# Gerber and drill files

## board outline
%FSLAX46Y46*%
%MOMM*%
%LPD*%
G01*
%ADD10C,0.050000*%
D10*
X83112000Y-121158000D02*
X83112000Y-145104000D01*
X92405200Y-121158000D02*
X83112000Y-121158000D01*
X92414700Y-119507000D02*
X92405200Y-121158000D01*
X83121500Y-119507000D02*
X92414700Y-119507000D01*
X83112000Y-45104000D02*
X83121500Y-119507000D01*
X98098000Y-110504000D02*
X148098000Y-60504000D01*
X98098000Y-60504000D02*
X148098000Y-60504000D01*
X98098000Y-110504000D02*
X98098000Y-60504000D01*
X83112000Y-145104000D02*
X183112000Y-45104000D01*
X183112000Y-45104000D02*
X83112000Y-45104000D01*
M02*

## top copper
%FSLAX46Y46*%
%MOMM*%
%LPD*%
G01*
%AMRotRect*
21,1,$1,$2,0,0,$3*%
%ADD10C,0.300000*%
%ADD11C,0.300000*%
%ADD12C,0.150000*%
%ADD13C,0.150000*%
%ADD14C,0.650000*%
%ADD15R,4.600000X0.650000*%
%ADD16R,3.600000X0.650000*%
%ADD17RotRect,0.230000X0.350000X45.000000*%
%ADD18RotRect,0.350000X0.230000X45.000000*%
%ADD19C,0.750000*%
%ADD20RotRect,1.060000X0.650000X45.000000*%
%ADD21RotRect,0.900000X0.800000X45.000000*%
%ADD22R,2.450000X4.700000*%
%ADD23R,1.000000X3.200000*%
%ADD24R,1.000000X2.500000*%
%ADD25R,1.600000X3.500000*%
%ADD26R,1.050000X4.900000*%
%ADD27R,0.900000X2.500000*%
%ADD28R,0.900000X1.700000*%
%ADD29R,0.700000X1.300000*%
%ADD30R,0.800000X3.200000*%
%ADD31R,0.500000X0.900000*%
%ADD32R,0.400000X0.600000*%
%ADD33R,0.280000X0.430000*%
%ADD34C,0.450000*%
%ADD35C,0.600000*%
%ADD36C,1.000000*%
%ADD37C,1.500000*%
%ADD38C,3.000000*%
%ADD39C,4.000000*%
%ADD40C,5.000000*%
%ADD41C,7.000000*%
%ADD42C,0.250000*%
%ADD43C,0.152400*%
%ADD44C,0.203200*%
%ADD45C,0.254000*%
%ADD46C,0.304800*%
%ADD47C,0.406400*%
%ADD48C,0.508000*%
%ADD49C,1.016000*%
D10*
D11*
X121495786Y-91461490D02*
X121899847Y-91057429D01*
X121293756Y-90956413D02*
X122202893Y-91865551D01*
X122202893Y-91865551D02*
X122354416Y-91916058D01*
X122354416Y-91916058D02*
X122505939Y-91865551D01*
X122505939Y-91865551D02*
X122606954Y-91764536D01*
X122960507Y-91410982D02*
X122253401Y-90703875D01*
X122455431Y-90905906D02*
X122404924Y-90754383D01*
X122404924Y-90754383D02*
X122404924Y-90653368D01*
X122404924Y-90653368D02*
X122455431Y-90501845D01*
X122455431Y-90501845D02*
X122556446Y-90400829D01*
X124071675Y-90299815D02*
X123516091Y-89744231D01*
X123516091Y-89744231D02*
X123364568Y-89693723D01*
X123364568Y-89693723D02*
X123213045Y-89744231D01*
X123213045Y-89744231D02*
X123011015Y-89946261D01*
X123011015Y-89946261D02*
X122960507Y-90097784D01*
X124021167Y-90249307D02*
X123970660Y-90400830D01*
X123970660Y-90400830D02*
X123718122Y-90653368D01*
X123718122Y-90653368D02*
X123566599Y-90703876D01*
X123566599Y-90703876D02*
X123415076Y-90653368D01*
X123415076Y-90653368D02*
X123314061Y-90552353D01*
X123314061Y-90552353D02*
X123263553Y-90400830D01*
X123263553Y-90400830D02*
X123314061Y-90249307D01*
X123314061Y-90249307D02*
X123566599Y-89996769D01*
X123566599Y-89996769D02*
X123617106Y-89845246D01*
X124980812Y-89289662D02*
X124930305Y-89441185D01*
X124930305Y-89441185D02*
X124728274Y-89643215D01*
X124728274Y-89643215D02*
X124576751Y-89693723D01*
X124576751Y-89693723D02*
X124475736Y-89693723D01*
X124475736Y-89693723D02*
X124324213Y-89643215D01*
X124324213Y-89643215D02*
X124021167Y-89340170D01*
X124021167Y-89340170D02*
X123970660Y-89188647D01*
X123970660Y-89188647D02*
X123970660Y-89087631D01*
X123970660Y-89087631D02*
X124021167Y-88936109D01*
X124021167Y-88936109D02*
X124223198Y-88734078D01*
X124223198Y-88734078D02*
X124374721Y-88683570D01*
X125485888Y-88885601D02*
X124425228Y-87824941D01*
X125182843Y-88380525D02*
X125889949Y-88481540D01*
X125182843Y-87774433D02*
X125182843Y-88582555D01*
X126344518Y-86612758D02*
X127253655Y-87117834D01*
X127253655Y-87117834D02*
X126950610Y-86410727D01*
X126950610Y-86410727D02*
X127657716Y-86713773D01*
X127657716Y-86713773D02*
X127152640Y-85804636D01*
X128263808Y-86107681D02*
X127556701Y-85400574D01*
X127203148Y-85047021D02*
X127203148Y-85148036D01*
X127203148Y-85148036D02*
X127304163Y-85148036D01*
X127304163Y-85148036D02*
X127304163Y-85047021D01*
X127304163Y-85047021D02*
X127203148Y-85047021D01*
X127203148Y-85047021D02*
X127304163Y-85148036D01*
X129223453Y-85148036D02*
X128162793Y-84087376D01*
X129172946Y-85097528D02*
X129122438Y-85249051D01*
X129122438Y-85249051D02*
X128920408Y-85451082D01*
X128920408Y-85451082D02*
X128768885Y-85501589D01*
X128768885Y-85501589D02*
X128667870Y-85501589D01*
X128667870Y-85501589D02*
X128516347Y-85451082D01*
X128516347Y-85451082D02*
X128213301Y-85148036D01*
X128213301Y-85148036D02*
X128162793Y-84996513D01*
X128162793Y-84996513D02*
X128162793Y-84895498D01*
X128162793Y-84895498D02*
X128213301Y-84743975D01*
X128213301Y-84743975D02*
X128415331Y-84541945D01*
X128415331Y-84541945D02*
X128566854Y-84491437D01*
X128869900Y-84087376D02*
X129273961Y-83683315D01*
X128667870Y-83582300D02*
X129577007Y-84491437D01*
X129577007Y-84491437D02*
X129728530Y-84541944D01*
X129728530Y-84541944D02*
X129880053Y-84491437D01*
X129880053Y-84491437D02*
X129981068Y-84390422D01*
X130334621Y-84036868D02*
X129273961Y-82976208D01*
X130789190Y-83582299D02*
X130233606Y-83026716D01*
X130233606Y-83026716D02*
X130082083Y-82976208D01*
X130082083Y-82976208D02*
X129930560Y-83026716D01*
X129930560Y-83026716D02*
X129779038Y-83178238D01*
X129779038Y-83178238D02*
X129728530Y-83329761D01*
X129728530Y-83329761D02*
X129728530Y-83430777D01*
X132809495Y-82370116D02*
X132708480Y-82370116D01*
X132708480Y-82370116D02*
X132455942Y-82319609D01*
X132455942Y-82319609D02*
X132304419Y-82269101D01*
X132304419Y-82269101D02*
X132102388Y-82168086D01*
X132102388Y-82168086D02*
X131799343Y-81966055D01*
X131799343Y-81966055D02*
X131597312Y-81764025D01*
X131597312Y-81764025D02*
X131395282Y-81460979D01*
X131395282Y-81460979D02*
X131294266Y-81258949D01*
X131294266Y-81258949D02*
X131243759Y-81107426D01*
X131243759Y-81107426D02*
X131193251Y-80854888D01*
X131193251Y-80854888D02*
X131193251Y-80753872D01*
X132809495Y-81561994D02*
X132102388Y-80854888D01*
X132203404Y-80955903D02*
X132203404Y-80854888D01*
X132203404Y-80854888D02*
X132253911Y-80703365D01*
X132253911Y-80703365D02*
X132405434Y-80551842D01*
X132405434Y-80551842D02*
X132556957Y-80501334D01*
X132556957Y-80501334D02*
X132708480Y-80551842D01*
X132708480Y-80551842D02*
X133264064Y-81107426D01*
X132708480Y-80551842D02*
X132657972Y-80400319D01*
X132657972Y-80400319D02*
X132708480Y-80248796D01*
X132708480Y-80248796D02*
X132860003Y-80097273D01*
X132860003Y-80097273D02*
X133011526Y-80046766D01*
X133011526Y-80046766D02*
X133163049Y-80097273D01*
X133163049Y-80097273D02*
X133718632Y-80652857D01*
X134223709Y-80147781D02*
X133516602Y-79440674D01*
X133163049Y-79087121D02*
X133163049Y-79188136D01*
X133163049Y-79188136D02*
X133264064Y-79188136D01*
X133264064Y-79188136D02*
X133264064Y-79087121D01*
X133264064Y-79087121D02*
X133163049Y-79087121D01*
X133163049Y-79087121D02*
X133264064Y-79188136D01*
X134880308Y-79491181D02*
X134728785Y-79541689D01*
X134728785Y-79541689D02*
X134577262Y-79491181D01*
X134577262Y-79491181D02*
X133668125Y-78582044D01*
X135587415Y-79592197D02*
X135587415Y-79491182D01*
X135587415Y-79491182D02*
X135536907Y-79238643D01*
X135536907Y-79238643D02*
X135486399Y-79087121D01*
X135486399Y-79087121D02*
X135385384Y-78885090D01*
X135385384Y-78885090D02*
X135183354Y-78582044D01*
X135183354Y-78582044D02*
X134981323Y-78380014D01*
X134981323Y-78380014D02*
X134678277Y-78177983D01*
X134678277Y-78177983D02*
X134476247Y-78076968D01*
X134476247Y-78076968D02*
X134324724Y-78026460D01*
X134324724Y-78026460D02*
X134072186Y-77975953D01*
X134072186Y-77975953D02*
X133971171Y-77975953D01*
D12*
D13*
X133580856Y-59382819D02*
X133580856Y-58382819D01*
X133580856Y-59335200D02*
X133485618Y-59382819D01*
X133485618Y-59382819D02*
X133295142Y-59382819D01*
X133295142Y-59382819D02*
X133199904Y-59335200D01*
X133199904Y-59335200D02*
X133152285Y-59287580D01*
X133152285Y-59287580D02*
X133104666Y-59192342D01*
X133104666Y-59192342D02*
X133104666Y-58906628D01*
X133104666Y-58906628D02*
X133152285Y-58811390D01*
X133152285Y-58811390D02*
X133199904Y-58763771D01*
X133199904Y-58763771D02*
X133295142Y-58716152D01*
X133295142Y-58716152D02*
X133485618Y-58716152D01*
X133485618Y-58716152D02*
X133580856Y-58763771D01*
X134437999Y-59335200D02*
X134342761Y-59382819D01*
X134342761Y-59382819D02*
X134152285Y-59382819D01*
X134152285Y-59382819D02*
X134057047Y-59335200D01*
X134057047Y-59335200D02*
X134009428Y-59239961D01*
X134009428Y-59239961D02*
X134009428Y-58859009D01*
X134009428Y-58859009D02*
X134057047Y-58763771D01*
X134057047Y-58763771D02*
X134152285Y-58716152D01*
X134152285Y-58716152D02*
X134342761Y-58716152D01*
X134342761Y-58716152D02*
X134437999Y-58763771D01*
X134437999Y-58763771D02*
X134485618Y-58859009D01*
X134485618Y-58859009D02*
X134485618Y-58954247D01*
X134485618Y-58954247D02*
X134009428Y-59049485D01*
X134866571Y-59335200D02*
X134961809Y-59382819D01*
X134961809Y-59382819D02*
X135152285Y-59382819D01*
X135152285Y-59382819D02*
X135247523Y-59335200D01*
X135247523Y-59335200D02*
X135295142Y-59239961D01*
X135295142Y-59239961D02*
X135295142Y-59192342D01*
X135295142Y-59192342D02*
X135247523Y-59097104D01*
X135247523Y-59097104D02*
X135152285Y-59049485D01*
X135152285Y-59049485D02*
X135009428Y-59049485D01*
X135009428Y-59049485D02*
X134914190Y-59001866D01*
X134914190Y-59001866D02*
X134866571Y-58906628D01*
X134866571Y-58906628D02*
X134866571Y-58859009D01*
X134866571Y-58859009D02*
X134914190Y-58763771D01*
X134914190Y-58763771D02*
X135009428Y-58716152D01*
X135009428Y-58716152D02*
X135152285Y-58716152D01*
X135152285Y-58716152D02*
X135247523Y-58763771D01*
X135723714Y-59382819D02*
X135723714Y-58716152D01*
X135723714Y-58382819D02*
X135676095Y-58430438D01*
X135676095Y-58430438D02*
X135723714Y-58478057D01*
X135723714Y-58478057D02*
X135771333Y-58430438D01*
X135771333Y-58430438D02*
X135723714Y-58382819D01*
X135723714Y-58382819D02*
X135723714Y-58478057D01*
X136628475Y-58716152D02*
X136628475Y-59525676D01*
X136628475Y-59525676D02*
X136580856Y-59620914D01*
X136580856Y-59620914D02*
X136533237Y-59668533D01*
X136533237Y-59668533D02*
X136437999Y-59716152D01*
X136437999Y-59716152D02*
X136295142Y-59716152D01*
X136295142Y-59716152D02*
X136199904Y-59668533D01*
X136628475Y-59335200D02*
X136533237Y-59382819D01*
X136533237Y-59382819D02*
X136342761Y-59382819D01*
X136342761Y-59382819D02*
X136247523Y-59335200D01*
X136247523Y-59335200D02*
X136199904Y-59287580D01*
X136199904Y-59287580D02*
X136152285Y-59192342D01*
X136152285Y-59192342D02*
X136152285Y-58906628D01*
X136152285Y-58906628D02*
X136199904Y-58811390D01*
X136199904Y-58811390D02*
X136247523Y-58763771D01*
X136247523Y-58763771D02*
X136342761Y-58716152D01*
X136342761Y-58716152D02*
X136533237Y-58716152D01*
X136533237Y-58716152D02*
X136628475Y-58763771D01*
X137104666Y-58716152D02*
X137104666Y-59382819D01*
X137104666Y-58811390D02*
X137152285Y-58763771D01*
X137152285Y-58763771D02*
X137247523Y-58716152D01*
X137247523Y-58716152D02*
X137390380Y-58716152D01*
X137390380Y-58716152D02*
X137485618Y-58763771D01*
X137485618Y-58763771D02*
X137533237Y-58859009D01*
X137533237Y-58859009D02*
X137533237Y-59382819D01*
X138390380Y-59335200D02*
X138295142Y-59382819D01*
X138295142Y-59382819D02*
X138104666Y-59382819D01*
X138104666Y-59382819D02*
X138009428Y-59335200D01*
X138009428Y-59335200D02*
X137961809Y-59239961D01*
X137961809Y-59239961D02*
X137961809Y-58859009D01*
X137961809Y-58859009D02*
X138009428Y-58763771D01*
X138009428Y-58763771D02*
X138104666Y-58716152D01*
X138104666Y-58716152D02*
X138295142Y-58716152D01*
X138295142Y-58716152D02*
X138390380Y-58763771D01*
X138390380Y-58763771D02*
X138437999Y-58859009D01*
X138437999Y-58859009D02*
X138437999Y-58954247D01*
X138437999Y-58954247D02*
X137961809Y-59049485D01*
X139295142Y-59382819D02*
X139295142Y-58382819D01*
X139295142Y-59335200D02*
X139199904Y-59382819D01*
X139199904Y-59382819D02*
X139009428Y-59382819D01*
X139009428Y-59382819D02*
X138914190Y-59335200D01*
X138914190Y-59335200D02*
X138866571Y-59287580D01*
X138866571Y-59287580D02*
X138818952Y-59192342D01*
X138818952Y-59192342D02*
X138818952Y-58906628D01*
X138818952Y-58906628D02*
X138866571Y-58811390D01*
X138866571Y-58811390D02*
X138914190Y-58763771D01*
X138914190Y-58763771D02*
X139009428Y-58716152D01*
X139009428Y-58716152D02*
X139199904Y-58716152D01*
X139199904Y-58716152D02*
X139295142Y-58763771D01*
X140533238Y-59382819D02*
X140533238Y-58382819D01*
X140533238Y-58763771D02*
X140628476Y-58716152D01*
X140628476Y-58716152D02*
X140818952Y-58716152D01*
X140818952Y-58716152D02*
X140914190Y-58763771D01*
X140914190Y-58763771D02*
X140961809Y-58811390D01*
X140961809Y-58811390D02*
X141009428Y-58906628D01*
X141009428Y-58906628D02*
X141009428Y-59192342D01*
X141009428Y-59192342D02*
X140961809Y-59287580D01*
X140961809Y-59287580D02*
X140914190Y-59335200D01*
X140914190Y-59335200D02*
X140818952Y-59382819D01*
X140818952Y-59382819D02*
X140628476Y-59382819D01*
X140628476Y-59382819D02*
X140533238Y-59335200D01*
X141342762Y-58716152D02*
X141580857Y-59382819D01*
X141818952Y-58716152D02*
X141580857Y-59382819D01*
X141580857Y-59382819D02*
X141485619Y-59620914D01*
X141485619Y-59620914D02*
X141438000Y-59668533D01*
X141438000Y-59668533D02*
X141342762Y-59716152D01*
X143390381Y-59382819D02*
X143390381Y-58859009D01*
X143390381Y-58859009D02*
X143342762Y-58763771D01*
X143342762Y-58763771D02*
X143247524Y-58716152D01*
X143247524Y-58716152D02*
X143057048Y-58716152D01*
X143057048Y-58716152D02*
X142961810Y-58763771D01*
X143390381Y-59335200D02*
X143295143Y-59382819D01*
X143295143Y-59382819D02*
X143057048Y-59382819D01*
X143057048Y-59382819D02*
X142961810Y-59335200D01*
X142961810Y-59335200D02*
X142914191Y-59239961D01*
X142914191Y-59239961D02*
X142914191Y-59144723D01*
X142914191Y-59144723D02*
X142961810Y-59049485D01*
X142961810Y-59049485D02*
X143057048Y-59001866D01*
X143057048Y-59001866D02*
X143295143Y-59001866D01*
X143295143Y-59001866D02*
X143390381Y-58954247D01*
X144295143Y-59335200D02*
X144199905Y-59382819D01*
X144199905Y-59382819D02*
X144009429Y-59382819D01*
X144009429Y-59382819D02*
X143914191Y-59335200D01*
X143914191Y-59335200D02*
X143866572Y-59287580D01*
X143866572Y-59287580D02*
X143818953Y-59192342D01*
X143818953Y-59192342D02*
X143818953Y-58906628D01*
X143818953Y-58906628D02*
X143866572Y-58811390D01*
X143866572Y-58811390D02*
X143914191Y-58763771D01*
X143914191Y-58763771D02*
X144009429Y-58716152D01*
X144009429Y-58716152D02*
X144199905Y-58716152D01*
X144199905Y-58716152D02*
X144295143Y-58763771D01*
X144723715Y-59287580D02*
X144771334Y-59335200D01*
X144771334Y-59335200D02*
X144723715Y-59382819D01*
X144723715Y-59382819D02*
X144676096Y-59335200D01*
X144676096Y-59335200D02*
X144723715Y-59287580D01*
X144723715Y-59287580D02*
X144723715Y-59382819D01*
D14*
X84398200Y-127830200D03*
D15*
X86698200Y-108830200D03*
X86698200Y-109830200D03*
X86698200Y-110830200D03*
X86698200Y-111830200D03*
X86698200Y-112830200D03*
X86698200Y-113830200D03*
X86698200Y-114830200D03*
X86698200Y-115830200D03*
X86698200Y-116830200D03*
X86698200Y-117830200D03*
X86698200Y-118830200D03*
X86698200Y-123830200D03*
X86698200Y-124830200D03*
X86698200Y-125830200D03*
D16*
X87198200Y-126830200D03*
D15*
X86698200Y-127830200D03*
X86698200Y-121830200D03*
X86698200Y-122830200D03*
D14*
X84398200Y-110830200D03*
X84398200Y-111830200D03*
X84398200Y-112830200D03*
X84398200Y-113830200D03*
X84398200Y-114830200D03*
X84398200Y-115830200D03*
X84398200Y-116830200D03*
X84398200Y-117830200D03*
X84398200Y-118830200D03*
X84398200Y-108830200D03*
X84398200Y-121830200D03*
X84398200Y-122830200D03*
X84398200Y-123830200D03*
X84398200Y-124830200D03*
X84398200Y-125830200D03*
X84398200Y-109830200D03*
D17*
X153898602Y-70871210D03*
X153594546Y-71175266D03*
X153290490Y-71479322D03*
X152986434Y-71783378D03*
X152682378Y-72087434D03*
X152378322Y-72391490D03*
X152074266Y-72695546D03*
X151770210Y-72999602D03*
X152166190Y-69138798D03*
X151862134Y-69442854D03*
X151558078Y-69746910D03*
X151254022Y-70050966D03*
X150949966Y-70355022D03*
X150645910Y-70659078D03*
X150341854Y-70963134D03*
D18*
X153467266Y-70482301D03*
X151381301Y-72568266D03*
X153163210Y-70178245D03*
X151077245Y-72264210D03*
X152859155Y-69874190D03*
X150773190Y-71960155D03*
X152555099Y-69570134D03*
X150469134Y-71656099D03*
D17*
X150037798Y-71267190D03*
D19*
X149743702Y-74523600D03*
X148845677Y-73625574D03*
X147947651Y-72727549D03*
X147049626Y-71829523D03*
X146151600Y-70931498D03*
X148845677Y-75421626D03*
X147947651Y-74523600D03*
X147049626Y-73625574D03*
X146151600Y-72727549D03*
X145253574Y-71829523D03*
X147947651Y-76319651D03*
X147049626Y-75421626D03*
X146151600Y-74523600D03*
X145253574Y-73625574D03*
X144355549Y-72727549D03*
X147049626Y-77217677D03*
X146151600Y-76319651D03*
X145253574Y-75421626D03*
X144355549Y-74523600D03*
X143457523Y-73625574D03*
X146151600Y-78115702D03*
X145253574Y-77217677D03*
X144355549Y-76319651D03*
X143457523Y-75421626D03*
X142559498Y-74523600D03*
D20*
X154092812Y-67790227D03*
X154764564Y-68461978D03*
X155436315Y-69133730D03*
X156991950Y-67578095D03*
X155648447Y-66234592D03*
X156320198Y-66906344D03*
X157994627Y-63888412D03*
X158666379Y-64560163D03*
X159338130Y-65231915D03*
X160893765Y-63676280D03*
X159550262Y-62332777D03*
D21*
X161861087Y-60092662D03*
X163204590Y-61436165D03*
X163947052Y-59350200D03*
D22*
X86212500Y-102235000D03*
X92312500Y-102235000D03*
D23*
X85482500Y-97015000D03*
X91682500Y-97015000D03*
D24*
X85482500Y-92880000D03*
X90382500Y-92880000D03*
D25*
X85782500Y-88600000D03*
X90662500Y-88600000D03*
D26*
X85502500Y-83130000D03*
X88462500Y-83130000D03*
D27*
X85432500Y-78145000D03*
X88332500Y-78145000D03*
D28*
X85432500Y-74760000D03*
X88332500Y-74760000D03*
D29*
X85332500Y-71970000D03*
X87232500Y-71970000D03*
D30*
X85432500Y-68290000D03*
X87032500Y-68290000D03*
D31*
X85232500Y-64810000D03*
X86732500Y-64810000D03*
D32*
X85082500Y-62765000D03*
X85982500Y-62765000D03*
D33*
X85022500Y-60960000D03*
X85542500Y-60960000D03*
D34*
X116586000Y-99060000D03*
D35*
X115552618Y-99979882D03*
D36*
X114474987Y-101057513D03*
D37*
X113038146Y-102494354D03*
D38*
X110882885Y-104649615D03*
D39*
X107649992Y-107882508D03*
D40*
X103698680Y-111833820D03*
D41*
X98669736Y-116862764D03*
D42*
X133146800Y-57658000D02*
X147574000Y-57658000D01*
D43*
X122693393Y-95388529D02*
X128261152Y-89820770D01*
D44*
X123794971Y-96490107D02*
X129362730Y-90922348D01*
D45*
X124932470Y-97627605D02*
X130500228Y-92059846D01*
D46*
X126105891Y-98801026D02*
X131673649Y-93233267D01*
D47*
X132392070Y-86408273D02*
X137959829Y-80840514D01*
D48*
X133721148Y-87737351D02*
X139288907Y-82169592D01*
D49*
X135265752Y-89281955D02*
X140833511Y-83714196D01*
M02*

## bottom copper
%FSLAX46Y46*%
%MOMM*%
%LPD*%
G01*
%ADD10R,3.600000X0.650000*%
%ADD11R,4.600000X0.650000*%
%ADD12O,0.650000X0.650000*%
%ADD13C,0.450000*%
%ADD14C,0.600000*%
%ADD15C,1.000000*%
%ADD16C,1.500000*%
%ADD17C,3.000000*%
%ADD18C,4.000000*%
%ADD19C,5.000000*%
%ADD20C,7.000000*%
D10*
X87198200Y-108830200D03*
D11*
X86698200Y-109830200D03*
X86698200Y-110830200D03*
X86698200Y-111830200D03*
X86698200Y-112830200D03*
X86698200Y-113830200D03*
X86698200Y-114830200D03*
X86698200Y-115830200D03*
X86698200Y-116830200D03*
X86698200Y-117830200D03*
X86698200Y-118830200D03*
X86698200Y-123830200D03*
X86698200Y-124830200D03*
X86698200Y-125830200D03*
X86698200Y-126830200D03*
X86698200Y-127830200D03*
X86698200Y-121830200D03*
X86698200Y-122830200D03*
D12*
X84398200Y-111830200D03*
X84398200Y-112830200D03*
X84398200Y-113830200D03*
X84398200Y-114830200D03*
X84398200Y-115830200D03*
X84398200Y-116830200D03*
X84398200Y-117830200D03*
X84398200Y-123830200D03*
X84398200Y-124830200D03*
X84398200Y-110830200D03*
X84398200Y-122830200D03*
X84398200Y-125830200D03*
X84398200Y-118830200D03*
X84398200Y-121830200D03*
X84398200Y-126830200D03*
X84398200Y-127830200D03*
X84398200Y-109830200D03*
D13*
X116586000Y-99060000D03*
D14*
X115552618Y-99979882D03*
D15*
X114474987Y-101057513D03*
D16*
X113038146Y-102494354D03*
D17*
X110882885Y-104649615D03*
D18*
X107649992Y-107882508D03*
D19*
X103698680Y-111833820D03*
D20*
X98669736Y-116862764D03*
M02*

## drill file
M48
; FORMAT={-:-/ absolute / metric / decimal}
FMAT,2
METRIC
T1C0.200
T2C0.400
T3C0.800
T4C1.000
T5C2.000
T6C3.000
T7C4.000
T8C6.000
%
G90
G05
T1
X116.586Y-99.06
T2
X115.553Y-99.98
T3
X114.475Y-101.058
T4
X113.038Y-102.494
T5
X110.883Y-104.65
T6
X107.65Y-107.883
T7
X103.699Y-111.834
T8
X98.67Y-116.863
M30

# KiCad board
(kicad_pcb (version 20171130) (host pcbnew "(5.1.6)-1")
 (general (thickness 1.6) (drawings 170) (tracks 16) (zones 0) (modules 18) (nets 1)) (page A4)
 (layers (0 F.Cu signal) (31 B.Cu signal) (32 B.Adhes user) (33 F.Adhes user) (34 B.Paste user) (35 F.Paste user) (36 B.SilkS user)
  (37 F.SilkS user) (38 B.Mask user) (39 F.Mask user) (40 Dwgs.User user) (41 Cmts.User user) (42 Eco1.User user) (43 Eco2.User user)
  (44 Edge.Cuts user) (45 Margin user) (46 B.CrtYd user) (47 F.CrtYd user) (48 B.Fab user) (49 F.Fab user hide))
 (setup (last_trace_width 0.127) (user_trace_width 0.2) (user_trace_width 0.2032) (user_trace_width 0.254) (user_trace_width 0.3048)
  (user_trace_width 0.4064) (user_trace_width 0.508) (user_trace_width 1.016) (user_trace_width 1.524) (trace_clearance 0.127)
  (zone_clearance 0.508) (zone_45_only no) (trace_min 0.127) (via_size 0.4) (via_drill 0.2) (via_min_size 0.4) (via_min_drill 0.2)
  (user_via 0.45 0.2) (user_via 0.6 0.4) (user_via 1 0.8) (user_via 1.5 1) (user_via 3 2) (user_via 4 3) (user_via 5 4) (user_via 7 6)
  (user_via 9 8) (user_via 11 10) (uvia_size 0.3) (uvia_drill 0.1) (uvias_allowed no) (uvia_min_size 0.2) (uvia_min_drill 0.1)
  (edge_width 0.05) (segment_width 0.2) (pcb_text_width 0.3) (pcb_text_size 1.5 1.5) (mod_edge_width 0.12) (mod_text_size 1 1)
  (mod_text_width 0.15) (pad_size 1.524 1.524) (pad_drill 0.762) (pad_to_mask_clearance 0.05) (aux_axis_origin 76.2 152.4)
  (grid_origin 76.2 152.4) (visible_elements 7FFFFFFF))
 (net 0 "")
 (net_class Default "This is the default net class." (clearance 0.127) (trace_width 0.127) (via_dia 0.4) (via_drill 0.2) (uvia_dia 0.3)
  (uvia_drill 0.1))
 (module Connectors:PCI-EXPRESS (layer F.Cu) (at 87.1982 108.8302 270)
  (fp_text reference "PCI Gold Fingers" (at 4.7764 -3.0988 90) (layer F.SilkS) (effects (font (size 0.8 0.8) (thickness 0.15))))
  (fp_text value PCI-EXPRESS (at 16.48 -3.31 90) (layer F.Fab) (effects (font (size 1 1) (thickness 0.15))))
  (pad "" connect circle (at 19 2.8 270) (size 0.65 0.65) (layers F.Cu F.Mask))
  (pad B1 connect rect (at 0 0.5 270) (size 0.65 4.6) (layers F.Cu F.Mask))
  (pad B2 connect rect (at 1 0.5 270) (size 0.65 4.6) (layers F.Cu F.Mask))
  (pad B3 connect rect (at 2 0.5 270) (size 0.65 4.6) (layers F.Cu F.Mask))
  (pad B4 connect rect (at 3 0.5 270) (size 0.65 4.6) (layers F.Cu F.Mask))
  (pad B5 connect rect (at 4 0.5 270) (size 0.65 4.6) (layers F.Cu F.Mask))
  (pad B6 connect rect (at 5 0.5 270) (size 0.65 4.6) (layers F.Cu F.Mask))
  (pad B7 connect rect (at 6 0.5 270) (size 0.65 4.6) (layers F.Cu F.Mask))
  (pad B8 connect rect (at 7 0.5 270) (size 0.65 4.6) (layers F.Cu F.Mask))
  (pad B9 connect rect (at 8 0.5 270) (size 0.65 4.6) (layers F.Cu F.Mask))
  (pad B10 connect rect (at 9 0.5 270) (size 0.65 4.6) (layers F.Cu F.Mask))
  (pad B11 connect rect (at 10 0.5 270) (size 0.65 4.6) (layers F.Cu F.Mask))
  (pad B14 connect rect (at 15 0.5 270) (size 0.65 4.6) (layers F.Cu F.Mask))
  (pad B15 connect rect (at 16 0.5 270) (size 0.65 4.6) (layers F.Cu F.Mask))
  (pad B16 connect rect (at 17 0.5 270) (size 0.65 4.6) (layers F.Cu F.Mask))
  (pad B17 connect rect (at 18 0 270) (size 0.65 3.6) (layers F.Cu F.Mask))
  (pad B18 connect rect (at 19 0.5 270) (size 0.65 4.6) (layers F.Cu F.Mask))
  (pad B12 connect rect (at 13 0.5 270) (size 0.65 4.6) (layers F.Cu F.Mask))
  (pad B13 connect rect (at 14 0.5 270) (size 0.65 4.6) (layers F.Cu F.Mask))
  (pad A1 connect rect (at 0 0 270) (size 0.65 3.6) (layers B.Cu B.Mask))
  (pad A2 connect rect (at 1 0.5 270) (size 0.65 4.6) (layers B.Cu B.Mask))
  (pad A3 connect rect (at 2 0.5 270) (size 0.65 4.6) (layers B.Cu B.Mask))
  (pad A4 connect rect (at 3 0.5 270) (size 0.65 4.6) (layers B.Cu B.Mask))
  (pad A5 connect rect (at 4 0.5 270) (size 0.65 4.6) (layers B.Cu B.Mask))
  (pad A6 connect rect (at 5 0.5 270) (size 0.65 4.6) (layers B.Cu B.Mask))
  (pad A7 connect rect (at 6 0.5 270) (size 0.65 4.6) (layers B.Cu B.Mask))
  (pad A8 connect rect (at 7 0.5 270) (size 0.65 4.6) (layers B.Cu B.Mask))
  (pad A9 connect rect (at 8 0.5 270) (size 0.65 4.6) (layers B.Cu B.Mask))
  (pad A10 connect rect (at 9 0.5 270) (size 0.65 4.6) (layers B.Cu B.Mask))
  (pad A11 connect rect (at 10 0.5 270) (size 0.65 4.6) (layers B.Cu B.Mask))
  (pad A14 connect rect (at 15 0.5 270) (size 0.65 4.6) (layers B.Cu B.Mask))
  (pad A15 connect rect (at 16 0.5 270) (size 0.65 4.6) (layers B.Cu B.Mask))
  (pad A16 connect rect (at 17 0.5 270) (size 0.65 4.6) (layers B.Cu B.Mask))
  (pad A17 connect rect (at 18 0.5 270) (size 0.65 4.6) (layers B.Cu B.Mask))
  (pad A18 connect rect (at 19 0.5 270) (size 0.65 4.6) (layers B.Cu B.Mask))
  (pad A12 connect rect (at 13 0.5 270) (size 0.65 4.6) (layers B.Cu B.Mask))
  (pad A13 connect rect (at 14 0.5 270) (size 0.65 4.6) (layers B.Cu B.Mask))
  (pad "" connect circle (at 2 2.8 270) (size 0.65 0.65) (layers F.Cu F.Mask))
  (pad "" connect circle (at 3 2.8 270) (size 0.65 0.65) (layers F.Cu F.Mask))
  (pad "" connect circle (at 4 2.8 270) (size 0.65 0.65) (layers F.Cu F.Mask))
  (pad "" connect circle (at 5 2.8 270) (size 0.65 0.65) (layers F.Cu F.Mask))
  (pad "" connect circle (at 6 2.8 270) (size 0.65 0.65) (layers F.Cu F.Mask))
  (pad "" connect circle (at 7 2.8 270) (size 0.65 0.65) (layers F.Cu F.Mask))
  (pad "" connect circle (at 8 2.8 270) (size 0.65 0.65) (layers F.Cu F.Mask))
  (pad "" connect circle (at 9 2.8 270) (size 0.65 0.65) (layers F.Cu F.Mask))
  (pad "" connect circle (at 10 2.8 270) (size 0.65 0.65) (layers F.Cu F.Mask))
  (pad "" connect circle (at 0 2.8 270) (size 0.65 0.65) (layers F.Cu F.Mask))
  (pad "" connect circle (at 13 2.8 270) (size 0.65 0.65) (layers F.Cu F.Mask))
  (pad "" connect circle (at 14 2.8 270) (size 0.65 0.65) (layers F.Cu F.Mask))
  (pad "" connect circle (at 15 2.8 270) (size 0.65 0.65) (layers F.Cu F.Mask))
  (pad "" connect circle (at 16 2.8 270) (size 0.65 0.65) (layers F.Cu F.Mask))
  (pad "" connect circle (at 17 2.8 270) (size 0.65 0.65) (layers F.Cu F.Mask))
  (pad "" connect circle (at 1 2.8 270) (size 0.65 0.65) (layers F.Cu F.Mask))
  (pad "" connect oval (at 3 2.8) (size 0.65 0.65) (layers B.Cu B.Mask))
  (pad "" connect oval (at 4 2.8) (size 0.65 0.65) (layers B.Cu B.Mask))
  (pad "" connect oval (at 5 2.8) (size 0.65 0.65) (layers B.Cu B.Mask))
  (pad "" connect oval (at 6 2.8) (size 0.65 0.65) (layers B.Cu B.Mask))
  (pad "" connect oval (at 7 2.8) (size 0.65 0.65) (layers B.Cu B.Mask))
  (pad "" connect oval (at 8 2.8) (size 0.65 0.65) (layers B.Cu B.Mask))
  (pad "" connect oval (at 9 2.8) (size 0.65 0.65) (layers B.Cu B.Mask))
  (pad "" connect oval (at 15 2.8) (size 0.65 0.65) (layers B.Cu B.Mask))
  (pad "" connect oval (at 16 2.8) (size 0.65 0.65) (layers B.Cu B.Mask))
  (pad "" connect oval (at 2 2.8) (size 0.65 0.65) (layers B.Cu B.Mask))
  (pad "" connect oval (at 14 2.8) (size 0.65 0.65) (layers B.Cu B.Mask))
  (pad "" connect oval (at 17 2.8) (size 0.65 0.65) (layers B.Cu B.Mask))
  (pad "" connect oval (at 10 2.8) (size 0.65 0.65) (layers B.Cu B.Mask))
  (pad "" connect oval (at 13 2.8) (size 0.65 0.65) (layers B.Cu B.Mask))
  (pad "" connect oval (at 18 2.8) (size 0.65 0.65) (layers B.Cu B.Mask))
  (pad "" connect oval (at 19 2.8) (size 0.65 0.65) (layers B.Cu B.Mask))
  (pad "" connect oval (at 1 2.8) (size 0.65 0.65) (layers B.Cu B.Mask)))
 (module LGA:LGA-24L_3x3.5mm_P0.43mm (layer F.Cu) (at 151.9682 71.0692 45)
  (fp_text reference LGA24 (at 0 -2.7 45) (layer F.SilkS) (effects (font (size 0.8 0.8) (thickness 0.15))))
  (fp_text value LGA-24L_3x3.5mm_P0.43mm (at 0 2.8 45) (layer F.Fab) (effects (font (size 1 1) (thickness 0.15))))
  (pad 13 smd rect (at 1.505 1.225 45) (size 0.23 0.35) (layers F.Cu F.Paste F.Mask))
  (pad 12 smd rect (at 1.075 1.225 45) (size 0.23 0.35) (layers F.Cu F.Paste F.Mask))
  (pad 11 smd rect (at 0.645 1.225 45) (size 0.23 0.35) (layers F.Cu F.Paste F.Mask))
  (pad 10 smd rect (at 0.215 1.225 45) (size 0.23 0.35) (layers F.Cu F.Paste F.Mask))
  (pad 9 smd rect (at -0.215 1.225 45) (size 0.23 0.35) (layers F.Cu F.Paste F.Mask))
  (pad 8 smd rect (at -0.645 1.225 45) (size 0.23 0.35) (layers F.Cu F.Paste F.Mask))
  (pad 7 smd rect (at -1.075 1.225 45) (size 0.23 0.35) (layers F.Cu F.Paste F.Mask))
  (pad 6 smd rect (at -1.505 1.225 45) (size 0.23 0.35) (layers F.Cu F.Paste F.Mask))
  (pad 18 smd rect (at 1.505 -1.225 45) (size 0.23 0.35) (layers F.Cu F.Paste F.Mask))
  (pad 19 smd rect (at 1.075 -1.225 45) (size 0.23 0.35) (layers F.Cu F.Paste F.Mask))
  (pad 20 smd rect (at 0.645 -1.225 45) (size 0.23 0.35) (layers F.Cu F.Paste F.Mask))
  (pad 21 smd rect (at 0.215 -1.225 45) (size 0.23 0.35) (layers F.Cu F.Paste F.Mask))
  (pad 22 smd rect (at -0.215 -1.225 45) (size 0.23 0.35) (layers F.Cu F.Paste F.Mask))
  (pad 23 smd rect (at -0.645 -1.225 45) (size 0.23 0.35) (layers F.Cu F.Paste F.Mask))
  (pad 24 smd rect (at -1.075 -1.225 45) (size 0.23 0.35) (layers F.Cu F.Paste F.Mask))
  (pad 14 smd rect (at 1.475 0.645 45) (size 0.35 0.23) (layers F.Cu F.Paste F.Mask))
  (pad 5 smd rect (at -1.475 0.645 45) (size 0.35 0.23) (layers F.Cu F.Paste F.Mask))
  (pad 15 smd rect (at 1.475 0.215 45) (size 0.35 0.23) (layers F.Cu F.Paste F.Mask))
  (pad 4 smd rect (at -1.475 0.215 45) (size 0.35 0.23) (layers F.Cu F.Paste F.Mask))
  (pad 16 smd rect (at 1.475 -0.215 45) (size 0.35 0.23) (layers F.Cu F.Paste F.Mask))
  (pad 3 smd rect (at -1.475 -0.215 45) (size 0.35 0.23) (layers F.Cu F.Paste F.Mask))
  (pad 17 smd rect (at 1.475 -0.645 45) (size 0.35 0.23) (layers F.Cu F.Paste F.Mask))
  (pad 2 smd rect (at -1.475 -0.645 45) (size 0.35 0.23) (layers F.Cu F.Paste F.Mask))
  (pad 1 smd rect (at -1.505 -1.225 45) (size 0.23 0.35) (layers F.Cu F.Paste F.Mask)))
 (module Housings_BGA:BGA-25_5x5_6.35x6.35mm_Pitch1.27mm (layer F.Cu) (at 146.1516 74.5236 45)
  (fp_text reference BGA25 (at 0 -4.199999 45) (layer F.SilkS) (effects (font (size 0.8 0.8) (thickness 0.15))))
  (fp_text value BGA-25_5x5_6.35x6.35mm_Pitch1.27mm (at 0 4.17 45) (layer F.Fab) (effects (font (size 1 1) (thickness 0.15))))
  (pad E5 smd circle (at 2.54 2.54 45) (size 0.75 0.75) (layers F.Cu F.Paste F.Mask))
  (pad D5 smd circle (at 2.54 1.27 45) (size 0.75 0.75) (layers F.Cu F.Paste F.Mask))
  (pad C5 smd circle (at 2.54 0 45) (size 0.75 0.75) (layers F.Cu F.Paste F.Mask))
  (pad B5 smd circle (at 2.54 -1.27 45) (size 0.75 0.75) (layers F.Cu F.Paste F.Mask))
  (pad A5 smd circle (at 2.54 -2.54 45) (size 0.75 0.75) (layers F.Cu F.Paste F.Mask))
  (pad E4 smd circle (at 1.27 2.54 45) (size 0.75 0.75) (layers F.Cu F.Paste F.Mask))
  (pad D4 smd circle (at 1.27 1.27 45) (size 0.75 0.75) (layers F.Cu F.Paste F.Mask))
  (pad C4 smd circle (at 1.27 0 45) (size 0.75 0.75) (layers F.Cu F.Paste F.Mask))
  (pad B4 smd circle (at 1.27 -1.27 45) (size 0.75 0.75) (layers F.Cu F.Paste F.Mask))
  (pad A4 smd circle (at 1.27 -2.54 45) (size 0.75 0.75) (layers F.Cu F.Paste F.Mask))
  (pad E3 smd circle (at 0 2.54 45) (size 0.75 0.75) (layers F.Cu F.Paste F.Mask))
  (pad D3 smd circle (at 0 1.27 45) (size 0.75 0.75) (layers F.Cu F.Paste F.Mask))
  (pad C3 smd circle (at 0 0 45) (size 0.75 0.75) (layers F.Cu F.Paste F.Mask))
  (pad B3 smd circle (at 0 -1.27 45) (size 0.75 0.75) (layers F.Cu F.Paste F.Mask))
  (pad A3 smd circle (at 0 -2.54 45) (size 0.75 0.75) (layers F.Cu F.Paste F.Mask))
  (pad E2 smd circle (at -1.27 2.54 45) (size 0.75 0.75) (layers F.Cu F.Paste F.Mask))
  (pad D2 smd circle (at -1.27 1.27 45) (size 0.75 0.75) (layers F.Cu F.Paste F.Mask))
  (pad C2 smd circle (at -1.27 0 45) (size 0.75 0.75) (layers F.Cu F.Paste F.Mask))
  (pad B2 smd circle (at -1.27 -1.27 45) (size 0.75 0.75) (layers F.Cu F.Paste F.Mask))
  (pad A2 smd circle (at -1.27 -2.54 45) (size 0.75 0.75) (layers F.Cu F.Paste F.Mask))
  (pad E1 smd circle (at -2.54 2.54 45) (size 0.75 0.75) (layers F.Cu F.Paste F.Mask))
  (pad D1 smd circle (at -2.54 1.27 45) (size 0.75 0.75) (layers F.Cu F.Paste F.Mask))
  (pad C1 smd circle (at -2.54 0 45) (size 0.75 0.75) (layers F.Cu F.Paste F.Mask))
  (pad B1 smd circle (at -2.54 -1.27 45) (size 0.75 0.75) (layers F.Cu F.Paste F.Mask))
  (pad A1 smd circle (at -2.54 -2.54 45) (size 0.75 0.75) (layers F.Cu F.Paste F.Mask)))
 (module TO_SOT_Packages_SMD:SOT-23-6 (layer F.Cu) (at 155.542381 67.684161 45)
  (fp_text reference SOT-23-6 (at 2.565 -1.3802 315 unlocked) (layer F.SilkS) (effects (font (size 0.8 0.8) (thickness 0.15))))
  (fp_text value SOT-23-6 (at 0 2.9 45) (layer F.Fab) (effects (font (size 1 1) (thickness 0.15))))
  (pad 1 smd rect (at -1.1 -0.95 45) (size 1.06 0.65) (layers F.Cu F.Paste F.Mask))
  (pad 2 smd rect (at -1.1 0 45) (size 1.06 0.65) (layers F.Cu F.Paste F.Mask))
  (pad 3 smd rect (at -1.1 0.95 45) (size 1.06 0.65) (layers F.Cu F.Paste F.Mask))
  (pad 4 smd rect (at 1.1 0.95 45) (size 1.06 0.65) (layers F.Cu F.Paste F.Mask))
  (pad 6 smd rect (at 1.1 -0.95 45) (size 1.06 0.65) (layers F.Cu F.Paste F.Mask))
  (pad 5 smd rect (at 1.1 0 45) (size 1.06 0.65) (layers F.Cu F.Paste F.Mask)))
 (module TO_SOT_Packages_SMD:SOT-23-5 (layer F.Cu) (at 159.444196 63.782346 45)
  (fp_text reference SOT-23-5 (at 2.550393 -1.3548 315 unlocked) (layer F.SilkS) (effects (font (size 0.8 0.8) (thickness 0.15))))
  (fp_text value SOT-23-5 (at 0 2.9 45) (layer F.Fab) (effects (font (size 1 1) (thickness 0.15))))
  (pad 1 smd rect (at -1.1 -0.95 45) (size 1.06 0.65) (layers F.Cu F.Paste F.Mask))
  (pad 2 smd rect (at -1.1 0 45) (size 1.06 0.65) (layers F.Cu F.Paste F.Mask))
  (pad 3 smd rect (at -1.1 0.95 45) (size 1.06 0.65) (layers F.Cu F.Paste F.Mask))
  (pad 4 smd rect (at 1.1 0.95 45) (size 1.06 0.65) (layers F.Cu F.Paste F.Mask))
  (pad 5 smd rect (at 1.1 -0.95 45) (size 1.06 0.65) (layers F.Cu F.Paste F.Mask)))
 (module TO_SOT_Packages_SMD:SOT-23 (layer F.Cu) (at 163.239945 60.057307 45)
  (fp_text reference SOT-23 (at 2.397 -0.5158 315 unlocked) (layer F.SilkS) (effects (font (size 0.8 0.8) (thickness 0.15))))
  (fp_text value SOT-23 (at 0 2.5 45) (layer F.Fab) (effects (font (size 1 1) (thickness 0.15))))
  (pad 1 smd rect (at -1 -0.95 45) (size 0.9 0.8) (layers F.Cu F.Paste F.Mask))
  (pad 2 smd rect (at -1 0.95 45) (size 0.9 0.8) (layers F.Cu F.Paste F.Mask))
  (pad 3 smd rect (at 1 0 45) (size 0.9 0.8) (layers F.Cu F.Paste F.Mask)))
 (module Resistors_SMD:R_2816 (layer F.Cu) (at 89.2625 102.235)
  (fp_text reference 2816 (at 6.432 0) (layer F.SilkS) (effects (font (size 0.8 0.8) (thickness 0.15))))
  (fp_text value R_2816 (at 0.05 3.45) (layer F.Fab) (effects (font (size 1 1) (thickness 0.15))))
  (pad 1 smd rect (at -3.05 0) (size 2.45 4.7) (layers F.Cu F.Paste F.Mask))
  (pad 2 smd rect (at 3.05 0) (size 2.45 4.7) (layers F.Cu F.Paste F.Mask)))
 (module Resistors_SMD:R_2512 (layer F.Cu) (at 88.5825 97.015)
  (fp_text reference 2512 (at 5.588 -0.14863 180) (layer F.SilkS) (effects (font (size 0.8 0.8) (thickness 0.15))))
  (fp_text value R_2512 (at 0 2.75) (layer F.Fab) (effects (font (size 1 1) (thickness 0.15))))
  (pad 1 smd rect (at -3.1 0) (size 1 3.2) (layers F.Cu F.Paste F.Mask))
  (pad 2 smd rect (at 3.1 0) (size 1 3.2) (layers F.Cu F.Paste F.Mask)))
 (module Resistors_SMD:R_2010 (layer F.Cu) (at 87.9325 92.88)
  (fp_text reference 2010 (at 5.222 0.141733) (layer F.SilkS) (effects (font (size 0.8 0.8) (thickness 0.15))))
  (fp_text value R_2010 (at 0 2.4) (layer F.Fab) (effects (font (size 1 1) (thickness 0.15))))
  (pad 1 smd rect (at -2.45 0) (size 1 2.5) (layers F.Cu F.Paste F.Mask))
  (pad 2 smd rect (at 2.45 0) (size 1 2.5) (layers F.Cu F.Paste F.Mask)))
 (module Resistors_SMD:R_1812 (layer F.Cu) (at 88.2225 88.6)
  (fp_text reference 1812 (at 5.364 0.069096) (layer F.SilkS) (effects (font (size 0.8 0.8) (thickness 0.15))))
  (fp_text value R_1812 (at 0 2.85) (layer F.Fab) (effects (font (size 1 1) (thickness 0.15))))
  (pad 1 smd rect (at -2.44 0) (size 1.6 3.5) (layers F.Cu F.Paste F.Mask))
  (pad 2 smd rect (at 2.44 0) (size 1.6 3.5) (layers F.Cu F.Paste F.Mask)))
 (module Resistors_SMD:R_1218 (layer F.Cu) (at 86.9825 83.13)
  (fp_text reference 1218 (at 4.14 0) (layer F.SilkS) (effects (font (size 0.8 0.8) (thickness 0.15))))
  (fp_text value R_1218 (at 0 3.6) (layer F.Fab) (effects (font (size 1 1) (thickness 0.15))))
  (pad 1 smd rect (at -1.48 0) (size 1.05 4.9) (layers F.Cu F.Paste F.Mask))
  (pad 2 smd rect (at 1.48 0) (size 1.05 4.9) (layers F.Cu F.Paste F.Mask)))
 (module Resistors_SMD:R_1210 (layer F.Cu) (at 86.8825 78.145)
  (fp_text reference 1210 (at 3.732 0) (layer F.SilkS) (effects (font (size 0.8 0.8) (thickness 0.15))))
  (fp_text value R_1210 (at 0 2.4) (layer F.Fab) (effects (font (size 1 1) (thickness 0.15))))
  (pad 1 smd rect (at -1.45 0) (size 0.9 2.5) (layers F.Cu F.Paste F.Mask))
  (pad 2 smd rect (at 1.45 0) (size 0.9 2.5) (layers F.Cu F.Paste F.Mask)))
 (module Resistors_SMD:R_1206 (layer F.Cu) (at 86.8825 74.76)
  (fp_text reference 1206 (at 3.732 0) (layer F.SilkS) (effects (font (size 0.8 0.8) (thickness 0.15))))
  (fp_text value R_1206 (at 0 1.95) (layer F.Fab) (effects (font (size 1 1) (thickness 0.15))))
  (pad 1 smd rect (at -1.45 0) (size 0.9 1.7) (layers F.Cu F.Paste F.Mask))
  (pad 2 smd rect (at 1.45 0) (size 0.9 1.7) (layers F.Cu F.Paste F.Mask)))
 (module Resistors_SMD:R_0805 (layer F.Cu) (at 86.2825 71.97)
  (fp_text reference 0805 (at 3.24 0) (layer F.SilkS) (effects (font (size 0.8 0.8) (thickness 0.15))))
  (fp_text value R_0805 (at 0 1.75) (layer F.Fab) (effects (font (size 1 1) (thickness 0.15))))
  (pad 1 smd rect (at -0.95 0) (size 0.7 1.3) (layers F.Cu F.Paste F.Mask))
  (pad 2 smd rect (at 0.95 0) (size 0.7 1.3) (layers F.Cu F.Paste F.Mask)))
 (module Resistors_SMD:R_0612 (layer F.Cu) (at 86.2325 68.29)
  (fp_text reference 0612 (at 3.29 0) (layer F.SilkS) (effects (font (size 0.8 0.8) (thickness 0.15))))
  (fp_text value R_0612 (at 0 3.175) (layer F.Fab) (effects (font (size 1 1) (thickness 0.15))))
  (pad 1 smd rect (at -0.8 0) (size 0.8 3.2) (layers F.Cu F.Paste F.Mask))
  (pad 2 smd rect (at 0.8 0) (size 0.8 3.2) (layers F.Cu F.Paste F.Mask)))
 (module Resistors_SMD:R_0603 (layer F.Cu) (at 85.9825 64.81)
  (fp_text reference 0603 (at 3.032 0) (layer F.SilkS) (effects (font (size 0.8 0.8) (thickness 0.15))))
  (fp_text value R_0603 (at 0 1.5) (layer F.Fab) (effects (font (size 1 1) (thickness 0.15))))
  (pad 1 smd rect (at -0.75 0) (size 0.5 0.9) (layers F.Cu F.Paste F.Mask))
  (pad 2 smd rect (at 0.75 0) (size 0.5 0.9) (layers F.Cu F.Paste F.Mask)))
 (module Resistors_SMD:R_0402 (layer F.Cu) (at 85.5325 62.765)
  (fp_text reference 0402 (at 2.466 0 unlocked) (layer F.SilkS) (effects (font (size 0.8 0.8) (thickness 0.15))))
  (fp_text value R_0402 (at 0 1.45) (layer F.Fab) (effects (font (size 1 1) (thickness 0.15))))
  (pad 1 smd rect (at -0.45 0) (size 0.4 0.6) (layers F.Cu F.Paste F.Mask))
  (pad 2 smd rect (at 0.45 0) (size 0.4 0.6) (layers F.Cu F.Paste F.Mask)))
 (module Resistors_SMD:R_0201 (layer F.Cu) (at 85.2825 60.96)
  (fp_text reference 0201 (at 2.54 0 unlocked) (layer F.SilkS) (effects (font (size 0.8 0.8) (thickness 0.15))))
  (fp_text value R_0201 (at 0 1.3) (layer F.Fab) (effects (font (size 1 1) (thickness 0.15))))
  (pad 1 smd rect (at -0.26 0) (size 0.28 0.43) (layers F.Cu F.Paste F.Mask))
  (pad 2 smd rect (at 0.26 0) (size 0.28 0.43) (layers F.Cu F.Paste F.Mask)))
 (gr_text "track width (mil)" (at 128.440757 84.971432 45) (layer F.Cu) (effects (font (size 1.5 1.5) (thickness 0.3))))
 (gr_line (start 83.112 121.158) (end 83.112 145.104) (layer Edge.Cuts) (width 0.05))
 (gr_line (start 92.4052 121.158) (end 83.112 121.158) (layer Edge.Cuts) (width 0.05))
 (gr_line (start 92.4147 119.507) (end 92.4052 121.158) (layer Edge.Cuts) (width 0.05))
 (gr_line (start 83.1215 119.507) (end 92.4147 119.507) (layer Edge.Cuts) (width 0.05))
 (gr_line (start 83.112 45.104) (end 83.1215 119.507) (layer Edge.Cuts) (width 0.05))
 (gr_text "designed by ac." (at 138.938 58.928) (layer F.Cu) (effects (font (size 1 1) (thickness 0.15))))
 (gr_line (start 98.098 110.504) (end 148.098 60.504) (layer Edge.Cuts) (width 0.05))
 (gr_line (start 98.098 60.504) (end 148.098 60.504) (layer Edge.Cuts) (width 0.05))
 (gr_line (start 98.098 110.504) (end 98.098 60.504) (layer Edge.Cuts) (width 0.05))
 (gr_line (start 83.112 145.104) (end 183.112 45.104) (layer Edge.Cuts) (width 0.05))
 (gr_line (start 183.112 45.104) (end 83.112 45.104) (layer Edge.Cuts) (width 0.05))
 (segment (start 133.1468 57.658) (end 147.574 57.658) (width 0.25) (layer F.Cu) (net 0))
 (segment (start 122.693393 95.388529) (end 128.261152 89.82077) (width 0.1524) (layer F.Cu) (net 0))
 (segment (start 123.794971 96.490107) (end 129.36273 90.922348) (width 0.2032) (layer F.Cu) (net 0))
 (segment (start 124.93247 97.627605) (end 130.500228 92.059846) (width 0.254) (layer F.Cu) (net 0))
 (segment (start 126.105891 98.801026) (end 131.673649 93.233267) (width 0.3048) (layer F.Cu) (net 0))
 (segment (start 132.39207 86.408273) (end 137.959829 80.840514) (width 0.4064) (layer F.Cu) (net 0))
 (segment (start 133.721148 87.737351) (end 139.288907 82.169592) (width 0.508) (layer F.Cu) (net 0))
 (segment (start 135.265752 89.281955) (end 140.833511 83.714196) (width 1.016) (layer F.Cu) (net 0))
 (via (at 116.586 99.06) (size 0.45) (drill 0.2) (layers F.Cu B.Cu) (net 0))
 (via (at 115.552618 99.979882) (size 0.6) (drill 0.4) (layers F.Cu B.Cu) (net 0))
 (via (at 114.474987 101.057513) (size 1) (drill 0.8) (layers F.Cu B.Cu) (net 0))
 (via (at 113.038146 102.494354) (size 1.5) (drill 1) (layers F.Cu B.Cu) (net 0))
 (via (at 110.882885 104.649615) (size 3) (drill 2) (layers F.Cu B.Cu) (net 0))
 (via (at 107.649992 107.882508) (size 4) (drill 3) (layers F.Cu B.Cu) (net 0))
 (via (at 103.69868 111.83382) (size 5) (drill 4) (layers F.Cu B.Cu) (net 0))
 (via (at 98.669736 116.862764) (size 7) (drill 6) (layers F.Cu B.Cu) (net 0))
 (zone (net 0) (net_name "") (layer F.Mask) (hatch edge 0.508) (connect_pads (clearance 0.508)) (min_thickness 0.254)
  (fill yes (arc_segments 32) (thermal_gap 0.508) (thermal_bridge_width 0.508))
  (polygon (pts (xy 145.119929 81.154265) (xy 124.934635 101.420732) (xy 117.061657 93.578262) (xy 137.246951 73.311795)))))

